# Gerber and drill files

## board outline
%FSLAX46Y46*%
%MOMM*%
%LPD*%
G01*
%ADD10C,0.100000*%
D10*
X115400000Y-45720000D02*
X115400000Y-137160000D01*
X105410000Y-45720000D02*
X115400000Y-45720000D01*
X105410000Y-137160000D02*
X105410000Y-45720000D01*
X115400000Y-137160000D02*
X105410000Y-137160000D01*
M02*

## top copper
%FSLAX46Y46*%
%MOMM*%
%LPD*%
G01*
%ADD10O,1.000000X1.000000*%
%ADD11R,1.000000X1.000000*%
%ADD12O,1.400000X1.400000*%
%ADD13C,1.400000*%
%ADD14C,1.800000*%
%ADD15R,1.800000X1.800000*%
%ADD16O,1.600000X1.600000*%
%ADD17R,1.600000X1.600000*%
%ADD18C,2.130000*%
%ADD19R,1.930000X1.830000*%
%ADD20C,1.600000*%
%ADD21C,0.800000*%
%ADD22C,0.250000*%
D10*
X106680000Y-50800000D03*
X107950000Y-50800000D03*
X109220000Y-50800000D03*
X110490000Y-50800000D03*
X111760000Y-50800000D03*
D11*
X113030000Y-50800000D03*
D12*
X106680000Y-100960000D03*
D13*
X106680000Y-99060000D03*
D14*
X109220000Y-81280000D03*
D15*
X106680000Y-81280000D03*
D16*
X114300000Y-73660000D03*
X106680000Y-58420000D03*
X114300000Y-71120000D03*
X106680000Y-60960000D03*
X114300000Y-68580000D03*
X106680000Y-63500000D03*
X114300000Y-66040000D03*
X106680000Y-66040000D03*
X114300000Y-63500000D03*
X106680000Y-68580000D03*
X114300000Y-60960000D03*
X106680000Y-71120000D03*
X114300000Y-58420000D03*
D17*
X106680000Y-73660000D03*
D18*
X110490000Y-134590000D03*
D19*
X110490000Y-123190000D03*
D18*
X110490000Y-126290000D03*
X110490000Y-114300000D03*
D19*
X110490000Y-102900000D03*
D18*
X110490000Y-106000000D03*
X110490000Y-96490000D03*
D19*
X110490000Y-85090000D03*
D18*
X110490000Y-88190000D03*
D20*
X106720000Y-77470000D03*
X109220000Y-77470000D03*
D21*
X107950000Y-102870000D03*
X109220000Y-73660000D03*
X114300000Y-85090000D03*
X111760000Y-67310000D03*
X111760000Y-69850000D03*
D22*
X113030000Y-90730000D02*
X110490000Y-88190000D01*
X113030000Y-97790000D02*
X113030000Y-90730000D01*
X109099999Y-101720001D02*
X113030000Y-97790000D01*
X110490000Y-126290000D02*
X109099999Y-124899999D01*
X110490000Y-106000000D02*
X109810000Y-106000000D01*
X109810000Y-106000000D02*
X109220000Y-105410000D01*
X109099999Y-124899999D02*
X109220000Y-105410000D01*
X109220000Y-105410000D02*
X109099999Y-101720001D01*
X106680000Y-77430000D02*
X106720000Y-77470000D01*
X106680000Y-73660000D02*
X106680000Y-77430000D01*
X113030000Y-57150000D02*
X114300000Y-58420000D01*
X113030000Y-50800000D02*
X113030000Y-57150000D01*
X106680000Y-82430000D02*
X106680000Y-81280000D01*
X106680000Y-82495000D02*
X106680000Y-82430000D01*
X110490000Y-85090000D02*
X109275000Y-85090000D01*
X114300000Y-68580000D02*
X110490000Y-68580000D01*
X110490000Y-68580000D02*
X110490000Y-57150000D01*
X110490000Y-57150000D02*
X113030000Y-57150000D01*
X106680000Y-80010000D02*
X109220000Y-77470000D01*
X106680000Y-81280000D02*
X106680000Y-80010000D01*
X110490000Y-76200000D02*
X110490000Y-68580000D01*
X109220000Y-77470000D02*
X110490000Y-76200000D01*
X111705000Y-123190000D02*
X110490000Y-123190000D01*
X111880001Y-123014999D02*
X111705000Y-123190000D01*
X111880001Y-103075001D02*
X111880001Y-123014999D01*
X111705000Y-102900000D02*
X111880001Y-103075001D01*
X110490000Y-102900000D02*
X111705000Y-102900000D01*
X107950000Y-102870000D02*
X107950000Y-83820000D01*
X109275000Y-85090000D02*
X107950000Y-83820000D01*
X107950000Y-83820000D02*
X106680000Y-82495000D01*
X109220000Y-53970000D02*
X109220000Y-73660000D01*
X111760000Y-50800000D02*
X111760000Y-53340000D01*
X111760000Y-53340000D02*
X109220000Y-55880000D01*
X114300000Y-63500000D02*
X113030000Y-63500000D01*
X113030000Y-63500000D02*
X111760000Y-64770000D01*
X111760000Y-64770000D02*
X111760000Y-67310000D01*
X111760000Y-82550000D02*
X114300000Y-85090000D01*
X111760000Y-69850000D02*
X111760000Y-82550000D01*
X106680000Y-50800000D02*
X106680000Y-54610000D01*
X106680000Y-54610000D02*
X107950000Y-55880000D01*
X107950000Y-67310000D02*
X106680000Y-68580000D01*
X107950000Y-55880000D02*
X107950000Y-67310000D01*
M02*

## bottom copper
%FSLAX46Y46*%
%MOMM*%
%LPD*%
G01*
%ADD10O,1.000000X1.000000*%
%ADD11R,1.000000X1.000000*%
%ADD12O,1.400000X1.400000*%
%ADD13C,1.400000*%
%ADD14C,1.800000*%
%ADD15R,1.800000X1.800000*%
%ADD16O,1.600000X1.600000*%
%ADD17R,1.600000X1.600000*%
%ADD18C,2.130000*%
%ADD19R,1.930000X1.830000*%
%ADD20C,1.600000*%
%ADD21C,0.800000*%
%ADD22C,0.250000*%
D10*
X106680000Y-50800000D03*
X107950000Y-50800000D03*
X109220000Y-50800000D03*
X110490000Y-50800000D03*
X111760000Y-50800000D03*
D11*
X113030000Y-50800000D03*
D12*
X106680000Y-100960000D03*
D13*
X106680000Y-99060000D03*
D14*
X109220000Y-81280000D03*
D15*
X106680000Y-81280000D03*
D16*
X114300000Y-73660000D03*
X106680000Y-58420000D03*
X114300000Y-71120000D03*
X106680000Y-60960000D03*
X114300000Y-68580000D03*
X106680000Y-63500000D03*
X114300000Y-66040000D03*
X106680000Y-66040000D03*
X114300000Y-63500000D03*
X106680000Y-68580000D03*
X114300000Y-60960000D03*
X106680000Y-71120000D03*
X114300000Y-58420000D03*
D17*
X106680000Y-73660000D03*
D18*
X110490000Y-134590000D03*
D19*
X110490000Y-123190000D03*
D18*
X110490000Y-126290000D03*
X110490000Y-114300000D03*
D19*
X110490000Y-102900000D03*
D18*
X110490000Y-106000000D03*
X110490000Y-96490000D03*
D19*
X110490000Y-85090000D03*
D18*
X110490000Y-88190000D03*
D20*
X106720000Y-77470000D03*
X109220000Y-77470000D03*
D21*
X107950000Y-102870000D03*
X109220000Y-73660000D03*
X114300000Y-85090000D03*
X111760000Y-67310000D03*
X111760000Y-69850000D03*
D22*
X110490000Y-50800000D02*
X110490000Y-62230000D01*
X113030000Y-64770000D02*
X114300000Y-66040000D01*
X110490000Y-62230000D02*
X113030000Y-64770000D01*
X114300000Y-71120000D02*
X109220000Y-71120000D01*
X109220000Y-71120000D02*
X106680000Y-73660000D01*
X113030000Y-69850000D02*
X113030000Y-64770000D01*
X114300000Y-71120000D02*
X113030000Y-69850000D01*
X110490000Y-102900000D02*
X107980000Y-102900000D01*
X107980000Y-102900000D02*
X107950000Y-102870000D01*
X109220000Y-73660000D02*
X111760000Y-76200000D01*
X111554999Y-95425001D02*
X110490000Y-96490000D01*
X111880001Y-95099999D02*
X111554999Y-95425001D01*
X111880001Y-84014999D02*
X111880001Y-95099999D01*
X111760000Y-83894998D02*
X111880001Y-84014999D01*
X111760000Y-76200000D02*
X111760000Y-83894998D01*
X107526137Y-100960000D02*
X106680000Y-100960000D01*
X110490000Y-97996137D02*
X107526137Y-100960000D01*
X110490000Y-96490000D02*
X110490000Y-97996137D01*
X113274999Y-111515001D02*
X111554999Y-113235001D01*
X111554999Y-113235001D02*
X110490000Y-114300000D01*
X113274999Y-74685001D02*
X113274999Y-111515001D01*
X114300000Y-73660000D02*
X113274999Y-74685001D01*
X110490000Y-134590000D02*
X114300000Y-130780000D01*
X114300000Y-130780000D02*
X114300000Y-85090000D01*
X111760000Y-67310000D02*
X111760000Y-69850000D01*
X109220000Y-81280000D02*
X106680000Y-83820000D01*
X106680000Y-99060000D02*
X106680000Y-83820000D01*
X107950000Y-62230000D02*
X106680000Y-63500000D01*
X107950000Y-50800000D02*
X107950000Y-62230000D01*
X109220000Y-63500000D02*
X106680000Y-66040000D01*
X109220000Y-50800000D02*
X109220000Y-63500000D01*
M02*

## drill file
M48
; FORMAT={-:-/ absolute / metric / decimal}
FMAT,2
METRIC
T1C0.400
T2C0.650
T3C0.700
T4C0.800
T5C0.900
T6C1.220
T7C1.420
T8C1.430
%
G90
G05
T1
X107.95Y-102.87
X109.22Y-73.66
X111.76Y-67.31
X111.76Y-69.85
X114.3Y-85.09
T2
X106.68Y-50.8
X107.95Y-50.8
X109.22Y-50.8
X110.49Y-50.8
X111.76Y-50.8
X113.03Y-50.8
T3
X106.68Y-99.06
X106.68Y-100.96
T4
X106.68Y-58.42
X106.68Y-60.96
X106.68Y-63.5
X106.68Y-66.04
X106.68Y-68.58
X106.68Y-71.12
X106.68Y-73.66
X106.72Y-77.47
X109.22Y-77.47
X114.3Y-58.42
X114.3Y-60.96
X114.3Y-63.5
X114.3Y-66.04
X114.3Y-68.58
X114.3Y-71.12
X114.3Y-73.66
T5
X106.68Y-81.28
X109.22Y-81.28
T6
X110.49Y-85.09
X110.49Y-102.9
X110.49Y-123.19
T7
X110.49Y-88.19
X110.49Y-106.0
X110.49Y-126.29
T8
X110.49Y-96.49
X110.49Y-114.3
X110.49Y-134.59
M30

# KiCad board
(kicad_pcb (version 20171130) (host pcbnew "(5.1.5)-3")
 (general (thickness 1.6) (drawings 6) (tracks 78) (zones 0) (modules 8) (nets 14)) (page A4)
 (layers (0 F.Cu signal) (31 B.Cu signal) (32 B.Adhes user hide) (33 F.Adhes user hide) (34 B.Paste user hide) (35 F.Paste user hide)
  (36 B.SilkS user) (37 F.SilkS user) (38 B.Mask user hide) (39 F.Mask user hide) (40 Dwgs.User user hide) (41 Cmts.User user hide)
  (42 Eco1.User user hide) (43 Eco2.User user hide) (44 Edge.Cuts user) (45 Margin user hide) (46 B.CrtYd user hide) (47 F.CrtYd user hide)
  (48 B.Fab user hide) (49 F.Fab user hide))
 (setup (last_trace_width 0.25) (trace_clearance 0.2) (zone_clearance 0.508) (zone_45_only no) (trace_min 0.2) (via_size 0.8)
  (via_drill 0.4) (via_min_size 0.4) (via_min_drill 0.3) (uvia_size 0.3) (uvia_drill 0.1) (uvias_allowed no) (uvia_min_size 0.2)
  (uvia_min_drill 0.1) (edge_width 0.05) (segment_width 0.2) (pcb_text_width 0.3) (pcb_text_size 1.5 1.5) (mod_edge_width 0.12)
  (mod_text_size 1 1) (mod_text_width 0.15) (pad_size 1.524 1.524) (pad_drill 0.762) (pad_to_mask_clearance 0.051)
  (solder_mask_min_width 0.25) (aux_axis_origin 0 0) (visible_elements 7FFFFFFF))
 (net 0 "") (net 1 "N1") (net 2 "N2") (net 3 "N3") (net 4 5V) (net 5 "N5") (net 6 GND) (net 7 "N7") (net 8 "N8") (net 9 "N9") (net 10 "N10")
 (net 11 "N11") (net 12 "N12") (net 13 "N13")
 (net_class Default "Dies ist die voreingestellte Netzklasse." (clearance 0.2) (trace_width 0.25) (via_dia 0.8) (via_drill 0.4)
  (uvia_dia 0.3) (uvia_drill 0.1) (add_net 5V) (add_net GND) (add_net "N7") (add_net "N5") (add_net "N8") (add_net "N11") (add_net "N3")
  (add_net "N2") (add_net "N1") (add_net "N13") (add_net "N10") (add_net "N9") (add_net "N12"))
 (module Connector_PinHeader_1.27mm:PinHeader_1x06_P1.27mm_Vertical (layer F.Cu) (at 113.03 50.8 270)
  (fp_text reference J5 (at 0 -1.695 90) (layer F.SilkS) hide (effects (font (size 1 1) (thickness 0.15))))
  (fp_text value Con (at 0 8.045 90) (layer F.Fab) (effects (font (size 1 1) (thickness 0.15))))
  (pad 6 thru_hole oval (at 0 6.35 270) (size 1 1) (drill 0.65) (layers *.Cu *.Mask) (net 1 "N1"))
  (pad 5 thru_hole oval (at 0 5.08 270) (size 1 1) (drill 0.65) (layers *.Cu *.Mask) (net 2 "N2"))
  (pad 4 thru_hole oval (at 0 3.81 270) (size 1 1) (drill 0.65) (layers *.Cu *.Mask) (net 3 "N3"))
  (pad 3 thru_hole oval (at 0 2.54 270) (size 1 1) (drill 0.65) (layers *.Cu *.Mask) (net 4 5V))
  (pad 2 thru_hole oval (at 0 1.27 270) (size 1 1) (drill 0.65) (layers *.Cu *.Mask) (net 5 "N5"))
  (pad 1 thru_hole rect (at 0 0 270) (size 1 1) (drill 0.65) (layers *.Cu *.Mask) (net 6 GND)))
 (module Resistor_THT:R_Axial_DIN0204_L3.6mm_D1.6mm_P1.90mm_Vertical (layer F.Cu) (at 106.68 99.06 270)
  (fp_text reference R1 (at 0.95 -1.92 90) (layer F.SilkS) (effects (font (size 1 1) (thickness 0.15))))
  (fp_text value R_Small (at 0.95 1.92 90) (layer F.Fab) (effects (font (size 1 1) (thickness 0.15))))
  (pad 2 thru_hole oval (at 1.9 0 270) (size 1.4 1.4) (drill 0.7) (layers *.Cu *.Mask) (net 5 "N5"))
  (pad 1 thru_hole circle (at 0 0 270) (size 1.4 1.4) (drill 0.7) (layers *.Cu *.Mask) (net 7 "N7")))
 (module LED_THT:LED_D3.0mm (layer F.Cu) (at 106.68 81.28)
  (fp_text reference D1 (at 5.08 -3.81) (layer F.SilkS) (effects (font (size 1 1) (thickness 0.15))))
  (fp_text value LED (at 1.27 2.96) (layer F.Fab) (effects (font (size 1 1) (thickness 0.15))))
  (pad 2 thru_hole circle (at 2.54 0) (size 1.8 1.8) (drill 0.9) (layers *.Cu *.Mask) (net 7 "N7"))
  (pad 1 thru_hole rect (at 0 0) (size 1.8 1.8) (drill 0.9) (layers *.Cu *.Mask) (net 6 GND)))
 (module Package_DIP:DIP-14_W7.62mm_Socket (layer B.Cu) (at 106.68 73.66)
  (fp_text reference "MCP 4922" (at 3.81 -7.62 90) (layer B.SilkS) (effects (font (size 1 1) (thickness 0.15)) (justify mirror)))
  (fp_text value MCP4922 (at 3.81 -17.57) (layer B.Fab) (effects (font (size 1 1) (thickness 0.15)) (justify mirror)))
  (pad 14 thru_hole oval (at 7.62 0) (size 1.6 1.6) (drill 0.8) (layers *.Cu *.Mask) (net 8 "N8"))
  (pad 7 thru_hole oval (at 0 -15.24) (size 1.6 1.6) (drill 0.8) (layers *.Cu *.Mask) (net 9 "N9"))
  (pad 13 thru_hole oval (at 7.62 -2.54) (size 1.6 1.6) (drill 0.8) (layers *.Cu *.Mask) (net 4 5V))
  (pad 6 thru_hole oval (at 0 -12.7) (size 1.6 1.6) (drill 0.8) (layers *.Cu *.Mask) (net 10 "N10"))
  (pad 12 thru_hole oval (at 7.62 -5.08) (size 1.6 1.6) (drill 0.8) (layers *.Cu *.Mask) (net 6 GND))
  (pad 5 thru_hole oval (at 0 -10.16) (size 1.6 1.6) (drill 0.8) (layers *.Cu *.Mask) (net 2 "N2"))
  (pad 11 thru_hole oval (at 7.62 -7.62) (size 1.6 1.6) (drill 0.8) (layers *.Cu *.Mask) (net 4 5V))
  (pad 4 thru_hole oval (at 0 -7.62) (size 1.6 1.6) (drill 0.8) (layers *.Cu *.Mask) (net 3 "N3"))
  (pad 10 thru_hole oval (at 7.62 -10.16) (size 1.6 1.6) (drill 0.8) (layers *.Cu *.Mask) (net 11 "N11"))
  (pad 3 thru_hole oval (at 0 -5.08) (size 1.6 1.6) (drill 0.8) (layers *.Cu *.Mask) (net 1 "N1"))
  (pad 9 thru_hole oval (at 7.62 -12.7) (size 1.6 1.6) (drill 0.8) (layers *.Cu *.Mask) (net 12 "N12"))
  (pad 2 thru_hole oval (at 0 -2.54) (size 1.6 1.6) (drill 0.8) (layers *.Cu *.Mask) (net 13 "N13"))
  (pad 8 thru_hole oval (at 7.62 -15.24) (size 1.6 1.6) (drill 0.8) (layers *.Cu *.Mask) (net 6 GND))
  (pad 1 thru_hole rect (at 0 0) (size 1.6 1.6) (drill 0.8) (layers *.Cu *.Mask) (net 4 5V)))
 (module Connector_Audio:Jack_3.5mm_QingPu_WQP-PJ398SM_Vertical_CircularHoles (layer F.Cu) (at 110.49 123.19)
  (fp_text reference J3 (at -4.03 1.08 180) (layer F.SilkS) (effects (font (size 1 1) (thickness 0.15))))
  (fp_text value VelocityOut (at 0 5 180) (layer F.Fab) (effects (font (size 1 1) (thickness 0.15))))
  (pad T thru_hole circle (at 0 11.4 180) (size 2.13 2.13) (drill 1.43) (layers *.Cu *.Mask) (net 11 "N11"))
  (pad S thru_hole rect (at 0 0 180) (size 1.93 1.83) (drill 1.22) (layers *.Cu *.Mask) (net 6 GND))
  (pad TN thru_hole circle (at 0 3.1 180) (size 2.13 2.13) (drill 1.42) (layers *.Cu *.Mask)))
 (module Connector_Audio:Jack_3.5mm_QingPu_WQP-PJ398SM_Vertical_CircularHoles (layer F.Cu) (at 110.49 102.9)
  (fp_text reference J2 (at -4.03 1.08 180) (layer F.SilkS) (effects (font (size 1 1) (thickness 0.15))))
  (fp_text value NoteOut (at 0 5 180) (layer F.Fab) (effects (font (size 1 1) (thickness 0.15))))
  (pad T thru_hole circle (at 0 11.4 180) (size 2.13 2.13) (drill 1.43) (layers *.Cu *.Mask) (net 8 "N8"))
  (pad S thru_hole rect (at 0 0 180) (size 1.93 1.83) (drill 1.22) (layers *.Cu *.Mask) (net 6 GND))
  (pad TN thru_hole circle (at 0 3.1 180) (size 2.13 2.13) (drill 1.42) (layers *.Cu *.Mask)))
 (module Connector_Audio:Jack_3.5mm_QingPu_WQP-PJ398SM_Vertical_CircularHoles (layer F.Cu) (at 110.49 85.09)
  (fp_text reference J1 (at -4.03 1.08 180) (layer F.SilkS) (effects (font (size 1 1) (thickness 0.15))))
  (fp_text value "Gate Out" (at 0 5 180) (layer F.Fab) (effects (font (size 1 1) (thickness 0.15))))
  (pad T thru_hole circle (at 0 11.4 180) (size 2.13 2.13) (drill 1.43) (layers *.Cu *.Mask) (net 5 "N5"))
  (pad S thru_hole rect (at 0 0 180) (size 1.93 1.83) (drill 1.22) (layers *.Cu *.Mask) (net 6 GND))
  (pad TN thru_hole circle (at 0 3.1 180) (size 2.13 2.13) (drill 1.42) (layers *.Cu *.Mask)))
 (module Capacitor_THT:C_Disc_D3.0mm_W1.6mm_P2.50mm (layer F.Cu) (at 109.22 77.47 180)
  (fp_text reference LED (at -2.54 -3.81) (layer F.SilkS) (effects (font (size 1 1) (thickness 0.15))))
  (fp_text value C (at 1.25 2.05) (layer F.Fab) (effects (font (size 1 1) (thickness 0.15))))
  (pad 2 thru_hole circle (at 2.5 0 180) (size 1.6 1.6) (drill 0.8) (layers *.Cu *.Mask) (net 4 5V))
  (pad 1 thru_hole circle (at 0 0 180) (size 1.6 1.6) (drill 0.8) (layers *.Cu *.Mask) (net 6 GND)))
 (gr_line (start 115.4 45.72) (end 115.4 137.16) (layer Edge.Cuts) (width 0.1))
 (gr_line (start 105.41 45.72) (end 115.4 45.72) (layer Edge.Cuts) (width 0.1))
 (gr_line (start 105.41 137.16) (end 105.41 45.72) (layer Edge.Cuts) (width 0.1))
 (gr_line (start 115.4 137.16) (end 105.41 137.16) (layer Edge.Cuts) (width 0.1))
 (segment (start 113.03 90.73) (end 110.49 88.19) (width 0.25) (layer F.Cu) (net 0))
 (segment (start 113.03 97.79) (end 113.03 90.73) (width 0.25) (layer F.Cu) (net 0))
 (segment (start 109.099999 101.720001) (end 113.03 97.79) (width 0.25) (layer F.Cu) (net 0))
 (segment (start 110.49 126.29) (end 109.099999 124.899999) (width 0.25) (layer F.Cu) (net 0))
 (segment (start 110.49 106) (end 109.81 106) (width 0.25) (layer F.Cu) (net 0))
 (segment (start 109.81 106) (end 109.22 105.41) (width 0.25) (layer F.Cu) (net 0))
 (segment (start 109.099999 124.899999) (end 109.22 105.41) (width 0.25) (layer F.Cu) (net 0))
 (segment (start 109.22 105.41) (end 109.099999 101.720001) (width 0.25) (layer F.Cu) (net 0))
 (segment (start 110.49 50.8) (end 110.49 62.23) (width 0.25) (layer B.Cu) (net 4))
 (segment (start 113.03 64.77) (end 114.3 66.04) (width 0.25) (layer B.Cu) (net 4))
 (segment (start 110.49 62.23) (end 113.03 64.77) (width 0.25) (layer B.Cu) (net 4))
 (segment (start 106.68 77.43) (end 106.72 77.47) (width 0.25) (layer F.Cu) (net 4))
 (segment (start 106.68 73.66) (end 106.68 77.43) (width 0.25) (layer F.Cu) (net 4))
 (segment (start 114.3 71.12) (end 109.22 71.12) (width 0.25) (layer B.Cu) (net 4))
 (segment (start 109.22 71.12) (end 106.68 73.66) (width 0.25) (layer B.Cu) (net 4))
 (segment (start 113.03 69.85) (end 113.03 64.77) (width 0.25) (layer B.Cu) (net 4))
 (segment (start 114.3 71.12) (end 113.03 69.85) (width 0.25) (layer B.Cu) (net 4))
 (segment (start 113.03 57.15) (end 114.3 58.42) (width 0.25) (layer F.Cu) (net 6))
 (segment (start 113.03 50.8) (end 113.03 57.15) (width 0.25) (layer F.Cu) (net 6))
 (segment (start 106.68 82.43) (end 106.68 81.28) (width 0.25) (layer F.Cu) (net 6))
 (segment (start 106.68 82.495) (end 106.68 82.43) (width 0.25) (layer F.Cu) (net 6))
 (segment (start 110.49 85.09) (end 109.275 85.09) (width 0.25) (layer F.Cu) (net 6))
 (segment (start 114.3 68.58) (end 110.49 68.58) (width 0.25) (layer F.Cu) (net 6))
 (segment (start 110.49 68.58) (end 110.49 57.15) (width 0.25) (layer F.Cu) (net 6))
 (segment (start 110.49 57.15) (end 113.03 57.15) (width 0.25) (layer F.Cu) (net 6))
 (segment (start 106.68 80.01) (end 109.22 77.47) (width 0.25) (layer F.Cu) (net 6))
 (segment (start 106.68 81.28) (end 106.68 80.01) (width 0.25) (layer F.Cu) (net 6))
 (segment (start 110.49 76.2) (end 110.49 68.58) (width 0.25) (layer F.Cu) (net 6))
 (segment (start 109.22 77.47) (end 110.49 76.2) (width 0.25) (layer F.Cu) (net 6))
 (segment (start 111.705 123.19) (end 110.49 123.19) (width 0.25) (layer F.Cu) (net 6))
 (segment (start 111.880001 123.014999) (end 111.705 123.19) (width 0.25) (layer F.Cu) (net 6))
 (segment (start 111.880001 103.075001) (end 111.880001 123.014999) (width 0.25) (layer F.Cu) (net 6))
 (segment (start 111.705 102.9) (end 111.880001 103.075001) (width 0.25) (layer F.Cu) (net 6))
 (segment (start 110.49 102.9) (end 111.705 102.9) (width 0.25) (layer F.Cu) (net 6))
 (via (at 107.95 102.87) (size 0.8) (drill 0.4) (layers F.Cu B.Cu) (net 6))
 (segment (start 110.49 102.9) (end 107.98 102.9) (width 0.25) (layer B.Cu) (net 6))
 (segment (start 107.98 102.9) (end 107.95 102.87) (width 0.25) (layer B.Cu) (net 6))
 (segment (start 107.95 102.87) (end 107.95 83.82) (width 0.25) (layer F.Cu) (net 6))
 (segment (start 109.275 85.09) (end 107.95 83.82) (width 0.25) (layer F.Cu) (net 6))
 (segment (start 107.95 83.82) (end 106.68 82.495) (width 0.25) (layer F.Cu) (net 6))
 (segment (start 109.22 53.97) (end 109.22 73.66) (width 0.25) (layer F.Cu) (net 5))
 (segment (start 111.76 50.8) (end 111.76 53.34) (width 0.25) (layer F.Cu) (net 5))
 (segment (start 111.76 53.34) (end 109.22 55.88) (width 0.25) (layer F.Cu) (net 5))
 (via (at 109.22 73.66) (size 0.8) (drill 0.4) (layers F.Cu B.Cu) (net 5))
 (segment (start 109.22 73.66) (end 111.76 76.2) (width 0.25) (layer B.Cu) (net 5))
 (segment (start 111.554999 95.425001) (end 110.49 96.49) (width 0.25) (layer B.Cu) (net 5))
 (segment (start 111.880001 95.099999) (end 111.554999 95.425001) (width 0.25) (layer B.Cu) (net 5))
 (segment (start 111.880001 84.014999) (end 111.880001 95.099999) (width 0.25) (layer B.Cu) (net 5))
 (segment (start 111.76 83.894998) (end 111.880001 84.014999) (width 0.25) (layer B.Cu) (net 5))
 (segment (start 111.76 76.2) (end 111.76 83.894998) (width 0.25) (layer B.Cu) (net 5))
 (segment (start 107.526137 100.96) (end 106.68 100.96) (width 0.25) (layer B.Cu) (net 5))
 (segment (start 110.49 97.996137) (end 107.526137 100.96) (width 0.25) (layer B.Cu) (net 5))
 (segment (start 110.49 96.49) (end 110.49 97.996137) (width 0.25) (layer B.Cu) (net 5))
 (segment (start 113.274999 111.515001) (end 111.554999 113.235001) (width 0.25) (layer B.Cu) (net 8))
 (segment (start 111.554999 113.235001) (end 110.49 114.3) (width 0.25) (layer B.Cu) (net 8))
 (segment (start 113.274999 74.685001) (end 113.274999 111.515001) (width 0.25) (layer B.Cu) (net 8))
 (segment (start 114.3 73.66) (end 113.274999 74.685001) (width 0.25) (layer B.Cu) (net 8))
 (segment (start 110.49 134.59) (end 114.3 130.78) (width 0.25) (layer B.Cu) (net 11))
 (segment (start 114.3 130.78) (end 114.3 85.09) (width 0.25) (layer B.Cu) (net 11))
 (via (at 114.3 85.09) (size 0.8) (drill 0.4) (layers F.Cu B.Cu) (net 11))
 (segment (start 114.3 63.5) (end 113.03 63.5) (width 0.25) (layer F.Cu) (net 11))
 (segment (start 113.03 63.5) (end 111.76 64.77) (width 0.25) (layer F.Cu) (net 11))
 (via (at 111.76 67.31) (size 0.8) (drill 0.4) (layers F.Cu B.Cu) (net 11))
 (segment (start 111.76 64.77) (end 111.76 67.31) (width 0.25) (layer F.Cu) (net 11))
 (segment (start 111.76 67.31) (end 111.76 69.85) (width 0.25) (layer B.Cu) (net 11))
 (via (at 111.76 69.85) (size 0.8) (drill 0.4) (layers F.Cu B.Cu) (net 11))
 (segment (start 111.76 82.55) (end 114.3 85.09) (width 0.25) (layer F.Cu) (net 11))
 (segment (start 111.76 69.85) (end 111.76 82.55) (width 0.25) (layer F.Cu) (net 11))
 (segment (start 109.22 81.28) (end 106.68 83.82) (width 0.25) (layer B.Cu) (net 7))
 (segment (start 106.68 99.06) (end 106.68 83.82) (width 0.25) (layer B.Cu) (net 7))
 (segment (start 107.95 62.23) (end 106.68 63.5) (width 0.25) (layer B.Cu) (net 2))
 (segment (start 107.95 50.8) (end 107.95 62.23) (width 0.25) (layer B.Cu) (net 2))
 (segment (start 109.22 63.5) (end 106.68 66.04) (width 0.25) (layer B.Cu) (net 3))
 (segment (start 109.22 50.8) (end 109.22 63.5) (width 0.25) (layer B.Cu) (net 3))
 (segment (start 106.68 50.8) (end 106.68 54.61) (width 0.25) (layer F.Cu) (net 1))
 (segment (start 106.68 54.61) (end 107.95 55.88) (width 0.25) (layer F.Cu) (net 1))
 (segment (start 107.95 67.31) (end 106.68 68.58) (width 0.25) (layer F.Cu) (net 1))
 (segment (start 107.95 55.88) (end 107.95 67.31) (width 0.25) (layer F.Cu) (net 1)))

